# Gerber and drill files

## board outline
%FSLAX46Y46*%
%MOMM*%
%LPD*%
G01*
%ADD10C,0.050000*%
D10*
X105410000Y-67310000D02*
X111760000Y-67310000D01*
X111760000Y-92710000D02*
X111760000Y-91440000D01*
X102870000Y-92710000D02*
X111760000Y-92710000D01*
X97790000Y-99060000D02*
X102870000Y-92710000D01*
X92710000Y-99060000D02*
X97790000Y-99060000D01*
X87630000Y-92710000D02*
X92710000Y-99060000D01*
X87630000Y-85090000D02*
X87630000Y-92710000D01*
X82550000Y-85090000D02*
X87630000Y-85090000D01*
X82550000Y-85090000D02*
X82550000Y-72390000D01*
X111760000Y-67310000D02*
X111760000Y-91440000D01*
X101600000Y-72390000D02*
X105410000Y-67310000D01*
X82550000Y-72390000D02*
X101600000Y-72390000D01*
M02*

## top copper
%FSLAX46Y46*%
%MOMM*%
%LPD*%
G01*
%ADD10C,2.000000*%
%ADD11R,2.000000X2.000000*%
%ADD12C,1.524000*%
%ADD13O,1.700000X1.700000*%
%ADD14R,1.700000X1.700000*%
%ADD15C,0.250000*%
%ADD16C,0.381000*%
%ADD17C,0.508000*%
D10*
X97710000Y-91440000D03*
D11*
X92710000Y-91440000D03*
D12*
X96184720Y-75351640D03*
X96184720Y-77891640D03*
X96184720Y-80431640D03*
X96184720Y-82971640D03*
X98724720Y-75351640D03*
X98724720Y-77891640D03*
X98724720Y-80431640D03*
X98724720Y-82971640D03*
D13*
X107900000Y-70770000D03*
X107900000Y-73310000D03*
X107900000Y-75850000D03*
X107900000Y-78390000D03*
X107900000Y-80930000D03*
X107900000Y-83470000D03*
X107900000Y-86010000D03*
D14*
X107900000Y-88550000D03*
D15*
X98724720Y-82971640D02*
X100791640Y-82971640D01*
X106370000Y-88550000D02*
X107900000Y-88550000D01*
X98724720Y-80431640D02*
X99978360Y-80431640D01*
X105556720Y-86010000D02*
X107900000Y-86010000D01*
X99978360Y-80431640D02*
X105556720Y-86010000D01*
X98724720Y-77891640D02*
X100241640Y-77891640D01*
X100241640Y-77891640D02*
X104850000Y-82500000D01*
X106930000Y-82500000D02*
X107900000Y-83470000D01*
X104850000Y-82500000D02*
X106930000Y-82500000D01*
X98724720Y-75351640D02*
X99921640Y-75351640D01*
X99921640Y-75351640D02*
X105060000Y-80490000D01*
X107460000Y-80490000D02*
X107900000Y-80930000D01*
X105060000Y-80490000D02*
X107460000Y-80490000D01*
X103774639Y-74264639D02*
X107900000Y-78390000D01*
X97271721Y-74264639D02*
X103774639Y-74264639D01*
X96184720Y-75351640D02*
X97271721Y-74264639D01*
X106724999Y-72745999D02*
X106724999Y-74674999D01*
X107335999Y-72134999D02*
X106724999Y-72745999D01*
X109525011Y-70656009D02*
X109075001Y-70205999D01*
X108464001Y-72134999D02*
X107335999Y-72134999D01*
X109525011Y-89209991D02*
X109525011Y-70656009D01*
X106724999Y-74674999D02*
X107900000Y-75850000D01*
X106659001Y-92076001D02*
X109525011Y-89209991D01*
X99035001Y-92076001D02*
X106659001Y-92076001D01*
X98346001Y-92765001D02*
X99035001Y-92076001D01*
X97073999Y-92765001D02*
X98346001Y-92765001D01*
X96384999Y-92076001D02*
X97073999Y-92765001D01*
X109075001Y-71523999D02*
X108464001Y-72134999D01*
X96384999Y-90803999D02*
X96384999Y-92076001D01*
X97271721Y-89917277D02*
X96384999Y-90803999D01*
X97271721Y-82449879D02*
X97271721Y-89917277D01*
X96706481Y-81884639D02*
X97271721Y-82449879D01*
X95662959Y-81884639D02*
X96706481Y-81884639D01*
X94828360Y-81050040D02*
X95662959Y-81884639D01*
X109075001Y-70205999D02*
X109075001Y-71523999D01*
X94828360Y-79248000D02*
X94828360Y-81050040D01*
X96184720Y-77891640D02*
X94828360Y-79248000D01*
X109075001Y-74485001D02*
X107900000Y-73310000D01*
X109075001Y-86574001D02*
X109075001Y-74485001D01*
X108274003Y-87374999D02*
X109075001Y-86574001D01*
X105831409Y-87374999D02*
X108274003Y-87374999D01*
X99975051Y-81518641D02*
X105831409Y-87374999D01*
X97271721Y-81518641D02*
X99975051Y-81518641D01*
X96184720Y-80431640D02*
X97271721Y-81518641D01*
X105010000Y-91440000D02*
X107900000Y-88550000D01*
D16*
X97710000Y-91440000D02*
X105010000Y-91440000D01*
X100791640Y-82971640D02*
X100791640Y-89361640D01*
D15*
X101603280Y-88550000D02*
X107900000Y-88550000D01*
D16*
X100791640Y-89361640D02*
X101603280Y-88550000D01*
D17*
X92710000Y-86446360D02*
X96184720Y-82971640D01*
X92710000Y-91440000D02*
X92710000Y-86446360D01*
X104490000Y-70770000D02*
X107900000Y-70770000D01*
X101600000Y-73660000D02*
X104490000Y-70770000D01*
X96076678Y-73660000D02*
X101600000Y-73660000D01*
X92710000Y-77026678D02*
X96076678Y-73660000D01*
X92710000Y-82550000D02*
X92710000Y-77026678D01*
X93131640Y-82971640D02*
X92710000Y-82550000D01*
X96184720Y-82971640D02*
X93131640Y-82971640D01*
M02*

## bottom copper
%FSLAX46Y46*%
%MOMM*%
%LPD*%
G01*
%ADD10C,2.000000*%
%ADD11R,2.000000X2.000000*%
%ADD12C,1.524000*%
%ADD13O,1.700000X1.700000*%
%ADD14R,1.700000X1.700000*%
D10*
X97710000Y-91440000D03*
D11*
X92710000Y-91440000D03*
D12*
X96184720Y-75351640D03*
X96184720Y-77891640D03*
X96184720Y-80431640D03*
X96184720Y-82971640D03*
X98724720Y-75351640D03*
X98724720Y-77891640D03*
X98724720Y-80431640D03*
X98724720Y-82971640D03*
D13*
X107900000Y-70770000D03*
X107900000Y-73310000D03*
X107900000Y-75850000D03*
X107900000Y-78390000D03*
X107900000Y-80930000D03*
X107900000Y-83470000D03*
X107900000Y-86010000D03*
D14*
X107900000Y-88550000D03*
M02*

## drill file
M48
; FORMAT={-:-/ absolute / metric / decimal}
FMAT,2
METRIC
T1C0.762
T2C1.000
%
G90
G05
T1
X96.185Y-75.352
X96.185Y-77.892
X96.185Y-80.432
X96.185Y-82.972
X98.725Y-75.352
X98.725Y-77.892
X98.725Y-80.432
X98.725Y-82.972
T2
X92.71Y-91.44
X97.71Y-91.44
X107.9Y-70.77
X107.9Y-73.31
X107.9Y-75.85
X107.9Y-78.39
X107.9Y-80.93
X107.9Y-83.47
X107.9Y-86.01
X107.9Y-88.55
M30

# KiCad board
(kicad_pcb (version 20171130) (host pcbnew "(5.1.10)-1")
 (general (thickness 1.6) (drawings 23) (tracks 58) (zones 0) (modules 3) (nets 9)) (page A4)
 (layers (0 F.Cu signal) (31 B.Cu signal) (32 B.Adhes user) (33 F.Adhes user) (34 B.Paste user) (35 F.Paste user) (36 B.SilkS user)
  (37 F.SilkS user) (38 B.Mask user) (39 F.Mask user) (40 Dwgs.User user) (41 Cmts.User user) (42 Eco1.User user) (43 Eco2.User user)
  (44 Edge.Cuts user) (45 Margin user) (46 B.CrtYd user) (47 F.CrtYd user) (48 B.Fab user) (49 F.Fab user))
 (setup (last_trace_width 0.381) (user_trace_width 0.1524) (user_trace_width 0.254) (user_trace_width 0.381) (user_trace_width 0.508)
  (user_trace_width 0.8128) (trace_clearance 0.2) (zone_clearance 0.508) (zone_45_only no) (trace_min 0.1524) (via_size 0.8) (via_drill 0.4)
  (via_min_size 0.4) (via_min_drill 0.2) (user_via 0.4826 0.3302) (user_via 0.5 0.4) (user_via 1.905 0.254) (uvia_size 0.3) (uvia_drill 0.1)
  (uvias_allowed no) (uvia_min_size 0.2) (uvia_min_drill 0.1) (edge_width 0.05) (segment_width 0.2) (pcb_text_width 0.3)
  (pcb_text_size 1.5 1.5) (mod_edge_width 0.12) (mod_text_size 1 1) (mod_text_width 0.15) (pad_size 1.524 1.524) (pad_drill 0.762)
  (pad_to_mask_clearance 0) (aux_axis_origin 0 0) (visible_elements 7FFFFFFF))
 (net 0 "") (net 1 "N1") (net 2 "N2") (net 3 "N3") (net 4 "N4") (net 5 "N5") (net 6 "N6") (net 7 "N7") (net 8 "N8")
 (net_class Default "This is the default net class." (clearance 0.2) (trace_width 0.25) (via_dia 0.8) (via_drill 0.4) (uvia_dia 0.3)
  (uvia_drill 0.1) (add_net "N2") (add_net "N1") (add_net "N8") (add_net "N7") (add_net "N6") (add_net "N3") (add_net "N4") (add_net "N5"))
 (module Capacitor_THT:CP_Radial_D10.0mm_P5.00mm (layer F.Cu) (at 92.71 91.44)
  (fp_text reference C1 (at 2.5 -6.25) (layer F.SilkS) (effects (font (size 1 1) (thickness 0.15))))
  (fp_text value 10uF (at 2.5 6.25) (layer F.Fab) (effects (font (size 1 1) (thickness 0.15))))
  (pad 2 thru_hole circle (at 5 0) (size 2 2) (drill 1) (layers *.Cu *.Mask) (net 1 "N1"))
  (pad 1 thru_hole rect (at 0 0) (size 2 2) (drill 1) (layers *.Cu *.Mask) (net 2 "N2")))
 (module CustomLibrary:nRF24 (layer F.Cu) (at 93.64472 77.89164)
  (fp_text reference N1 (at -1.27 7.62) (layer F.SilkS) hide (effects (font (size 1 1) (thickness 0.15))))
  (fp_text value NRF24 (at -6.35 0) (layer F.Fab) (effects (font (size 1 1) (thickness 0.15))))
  (pad 4 thru_hole circle (at 2.54 -2.54) (size 1.524 1.524) (drill 0.762) (layers *.Cu *.Mask) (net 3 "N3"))
  (pad 5 thru_hole circle (at 2.54 0) (size 1.524 1.524) (drill 0.762) (layers *.Cu *.Mask) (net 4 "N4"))
  (pad 6 thru_hole circle (at 2.54 2.54) (size 1.524 1.524) (drill 0.762) (layers *.Cu *.Mask) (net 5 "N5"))
  (pad 7 thru_hole circle (at 2.54 5.08) (size 1.524 1.524) (drill 0.762) (layers *.Cu *.Mask) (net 2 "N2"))
  (pad 3 thru_hole circle (at 5.08 -2.54) (size 1.524 1.524) (drill 0.762) (layers *.Cu *.Mask) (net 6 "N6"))
  (pad 2 thru_hole circle (at 5.08 0) (size 1.524 1.524) (drill 0.762) (layers *.Cu *.Mask) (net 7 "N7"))
  (pad 1 thru_hole circle (at 5.08 2.54) (size 1.524 1.524) (drill 0.762) (layers *.Cu *.Mask) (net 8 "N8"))
  (pad 0 thru_hole circle (at 5.08 5.08) (size 1.524 1.524) (drill 0.762) (layers *.Cu *.Mask) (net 1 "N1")))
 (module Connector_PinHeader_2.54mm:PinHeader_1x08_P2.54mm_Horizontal (layer B.Cu) (at 107.9 88.55)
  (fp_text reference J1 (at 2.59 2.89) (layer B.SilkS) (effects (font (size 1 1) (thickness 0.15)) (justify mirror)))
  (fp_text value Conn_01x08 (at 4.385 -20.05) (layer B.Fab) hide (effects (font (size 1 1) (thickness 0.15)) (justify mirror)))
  (pad 8 thru_hole oval (at 0 -17.78) (size 1.7 1.7) (drill 1) (layers *.Cu *.Mask) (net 2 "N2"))
  (pad 7 thru_hole oval (at 0 -15.24) (size 1.7 1.7) (drill 1) (layers *.Cu *.Mask) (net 5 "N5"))
  (pad 6 thru_hole oval (at 0 -12.7) (size 1.7 1.7) (drill 1) (layers *.Cu *.Mask) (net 4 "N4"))
  (pad 5 thru_hole oval (at 0 -10.16) (size 1.7 1.7) (drill 1) (layers *.Cu *.Mask) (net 3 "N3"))
  (pad 4 thru_hole oval (at 0 -7.62) (size 1.7 1.7) (drill 1) (layers *.Cu *.Mask) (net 6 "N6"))
  (pad 3 thru_hole oval (at 0 -5.08) (size 1.7 1.7) (drill 1) (layers *.Cu *.Mask) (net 7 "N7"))
  (pad 2 thru_hole oval (at 0 -2.54) (size 1.7 1.7) (drill 1) (layers *.Cu *.Mask) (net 8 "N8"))
  (pad 1 thru_hole rect (at 0 0) (size 1.7 1.7) (drill 1) (layers *.Cu *.Mask) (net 1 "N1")))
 (gr_line (start 105.41 67.31) (end 111.76 67.31) (layer Edge.Cuts) (width 0.05))
 (gr_line (start 111.76 92.71) (end 111.76 91.44) (layer Edge.Cuts) (width 0.05))
 (gr_line (start 102.87 92.71) (end 111.76 92.71) (layer Edge.Cuts) (width 0.05))
 (gr_line (start 97.79 99.06) (end 102.87 92.71) (layer Edge.Cuts) (width 0.05))
 (gr_line (start 92.71 99.06) (end 97.79 99.06) (layer Edge.Cuts) (width 0.05))
 (gr_line (start 87.63 92.71) (end 92.71 99.06) (layer Edge.Cuts) (width 0.05))
 (gr_line (start 87.63 85.09) (end 87.63 92.71) (layer Edge.Cuts) (width 0.05))
 (gr_line (start 82.55 85.09) (end 87.63 85.09) (layer Edge.Cuts) (width 0.05))
 (gr_line (start 82.55 85.09) (end 82.55 72.39) (layer Edge.Cuts) (width 0.05))
 (gr_line (start 111.76 67.31) (end 111.76 91.44) (layer Edge.Cuts) (width 0.05))
 (gr_line (start 101.6 72.39) (end 105.41 67.31) (layer Edge.Cuts) (width 0.05))
 (gr_line (start 82.55 72.39) (end 101.6 72.39) (layer Edge.Cuts) (width 0.05))
 (segment (start 98.72472 82.97164) (end 100.79164 82.97164) (width 0.25) (layer F.Cu) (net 1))
 (segment (start 106.37 88.55) (end 107.9 88.55) (width 0.25) (layer F.Cu) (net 1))
 (segment (start 98.72472 80.43164) (end 99.97836 80.43164) (width 0.25) (layer F.Cu) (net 8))
 (segment (start 105.55672 86.01) (end 107.9 86.01) (width 0.25) (layer F.Cu) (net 8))
 (segment (start 99.97836 80.43164) (end 105.55672 86.01) (width 0.25) (layer F.Cu) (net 8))
 (segment (start 98.72472 77.89164) (end 100.24164 77.89164) (width 0.25) (layer F.Cu) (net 7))
 (segment (start 100.24164 77.89164) (end 104.85 82.5) (width 0.25) (layer F.Cu) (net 7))
 (segment (start 106.93 82.5) (end 107.9 83.47) (width 0.25) (layer F.Cu) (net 7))
 (segment (start 104.85 82.5) (end 106.93 82.5) (width 0.25) (layer F.Cu) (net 7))
 (segment (start 98.72472 75.35164) (end 99.92164 75.35164) (width 0.25) (layer F.Cu) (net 6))
 (segment (start 99.92164 75.35164) (end 105.06 80.49) (width 0.25) (layer F.Cu) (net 6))
 (segment (start 107.46 80.49) (end 107.9 80.93) (width 0.25) (layer F.Cu) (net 6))
 (segment (start 105.06 80.49) (end 107.46 80.49) (width 0.25) (layer F.Cu) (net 6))
 (segment (start 103.774639 74.264639) (end 107.9 78.39) (width 0.25) (layer F.Cu) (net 3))
 (segment (start 97.271721 74.264639) (end 103.774639 74.264639) (width 0.25) (layer F.Cu) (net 3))
 (segment (start 96.18472 75.35164) (end 97.271721 74.264639) (width 0.25) (layer F.Cu) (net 3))
 (segment (start 106.724999 72.745999) (end 106.724999 74.674999) (width 0.25) (layer F.Cu) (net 4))
 (segment (start 107.335999 72.134999) (end 106.724999 72.745999) (width 0.25) (layer F.Cu) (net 4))
 (segment (start 109.525011 70.656009) (end 109.075001 70.205999) (width 0.25) (layer F.Cu) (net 4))
 (segment (start 108.464001 72.134999) (end 107.335999 72.134999) (width 0.25) (layer F.Cu) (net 4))
 (segment (start 109.525011 89.209991) (end 109.525011 70.656009) (width 0.25) (layer F.Cu) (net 4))
 (segment (start 106.724999 74.674999) (end 107.9 75.85) (width 0.25) (layer F.Cu) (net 4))
 (segment (start 106.659001 92.076001) (end 109.525011 89.209991) (width 0.25) (layer F.Cu) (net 4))
 (segment (start 99.035001 92.076001) (end 106.659001 92.076001) (width 0.25) (layer F.Cu) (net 4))
 (segment (start 98.346001 92.765001) (end 99.035001 92.076001) (width 0.25) (layer F.Cu) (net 4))
 (segment (start 97.073999 92.765001) (end 98.346001 92.765001) (width 0.25) (layer F.Cu) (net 4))
 (segment (start 96.384999 92.076001) (end 97.073999 92.765001) (width 0.25) (layer F.Cu) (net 4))
 (segment (start 109.075001 71.523999) (end 108.464001 72.134999) (width 0.25) (layer F.Cu) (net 4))
 (segment (start 96.384999 90.803999) (end 96.384999 92.076001) (width 0.25) (layer F.Cu) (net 4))
 (segment (start 97.271721 89.917277) (end 96.384999 90.803999) (width 0.25) (layer F.Cu) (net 4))
 (segment (start 97.271721 82.449879) (end 97.271721 89.917277) (width 0.25) (layer F.Cu) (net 4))
 (segment (start 96.706481 81.884639) (end 97.271721 82.449879) (width 0.25) (layer F.Cu) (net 4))
 (segment (start 95.662959 81.884639) (end 96.706481 81.884639) (width 0.25) (layer F.Cu) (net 4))
 (segment (start 94.82836 81.05004) (end 95.662959 81.884639) (width 0.25) (layer F.Cu) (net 4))
 (segment (start 109.075001 70.205999) (end 109.075001 71.523999) (width 0.25) (layer F.Cu) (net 4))
 (segment (start 94.82836 79.248) (end 94.82836 81.05004) (width 0.25) (layer F.Cu) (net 4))
 (segment (start 96.18472 77.89164) (end 94.82836 79.248) (width 0.25) (layer F.Cu) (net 4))
 (segment (start 109.075001 74.485001) (end 107.9 73.31) (width 0.25) (layer F.Cu) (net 5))
 (segment (start 109.075001 86.574001) (end 109.075001 74.485001) (width 0.25) (layer F.Cu) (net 5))
 (segment (start 108.274003 87.374999) (end 109.075001 86.574001) (width 0.25) (layer F.Cu) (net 5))
 (segment (start 105.831409 87.374999) (end 108.274003 87.374999) (width 0.25) (layer F.Cu) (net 5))
 (segment (start 99.975051 81.518641) (end 105.831409 87.374999) (width 0.25) (layer F.Cu) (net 5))
 (segment (start 97.271721 81.518641) (end 99.975051 81.518641) (width 0.25) (layer F.Cu) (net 5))
 (segment (start 96.18472 80.43164) (end 97.271721 81.518641) (width 0.25) (layer F.Cu) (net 5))
 (segment (start 105.01 91.44) (end 107.9 88.55) (width 0.25) (layer F.Cu) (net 1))
 (segment (start 97.71 91.44) (end 105.01 91.44) (width 0.381) (layer F.Cu) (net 1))
 (segment (start 100.79164 82.97164) (end 100.79164 89.36164) (width 0.381) (layer F.Cu) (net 1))
 (segment (start 101.60328 88.55) (end 107.9 88.55) (width 0.25) (layer F.Cu) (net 1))
 (segment (start 100.79164 89.36164) (end 101.60328 88.55) (width 0.381) (layer F.Cu) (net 1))
 (segment (start 92.71 86.44636) (end 96.18472 82.97164) (width 0.508) (layer F.Cu) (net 2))
 (segment (start 92.71 91.44) (end 92.71 86.44636) (width 0.508) (layer F.Cu) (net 2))
 (segment (start 104.49 70.77) (end 107.9 70.77) (width 0.508) (layer F.Cu) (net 2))
 (segment (start 101.6 73.66) (end 104.49 70.77) (width 0.508) (layer F.Cu) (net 2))
 (segment (start 96.076678 73.66) (end 101.6 73.66) (width 0.508) (layer F.Cu) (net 2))
 (segment (start 92.71 77.026678) (end 96.076678 73.66) (width 0.508) (layer F.Cu) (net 2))
 (segment (start 92.71 82.55) (end 92.71 77.026678) (width 0.508) (layer F.Cu) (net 2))
 (segment (start 93.13164 82.97164) (end 92.71 82.55) (width 0.508) (layer F.Cu) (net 2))
 (segment (start 96.18472 82.97164) (end 93.13164 82.97164) (width 0.508) (layer F.Cu) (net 2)))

